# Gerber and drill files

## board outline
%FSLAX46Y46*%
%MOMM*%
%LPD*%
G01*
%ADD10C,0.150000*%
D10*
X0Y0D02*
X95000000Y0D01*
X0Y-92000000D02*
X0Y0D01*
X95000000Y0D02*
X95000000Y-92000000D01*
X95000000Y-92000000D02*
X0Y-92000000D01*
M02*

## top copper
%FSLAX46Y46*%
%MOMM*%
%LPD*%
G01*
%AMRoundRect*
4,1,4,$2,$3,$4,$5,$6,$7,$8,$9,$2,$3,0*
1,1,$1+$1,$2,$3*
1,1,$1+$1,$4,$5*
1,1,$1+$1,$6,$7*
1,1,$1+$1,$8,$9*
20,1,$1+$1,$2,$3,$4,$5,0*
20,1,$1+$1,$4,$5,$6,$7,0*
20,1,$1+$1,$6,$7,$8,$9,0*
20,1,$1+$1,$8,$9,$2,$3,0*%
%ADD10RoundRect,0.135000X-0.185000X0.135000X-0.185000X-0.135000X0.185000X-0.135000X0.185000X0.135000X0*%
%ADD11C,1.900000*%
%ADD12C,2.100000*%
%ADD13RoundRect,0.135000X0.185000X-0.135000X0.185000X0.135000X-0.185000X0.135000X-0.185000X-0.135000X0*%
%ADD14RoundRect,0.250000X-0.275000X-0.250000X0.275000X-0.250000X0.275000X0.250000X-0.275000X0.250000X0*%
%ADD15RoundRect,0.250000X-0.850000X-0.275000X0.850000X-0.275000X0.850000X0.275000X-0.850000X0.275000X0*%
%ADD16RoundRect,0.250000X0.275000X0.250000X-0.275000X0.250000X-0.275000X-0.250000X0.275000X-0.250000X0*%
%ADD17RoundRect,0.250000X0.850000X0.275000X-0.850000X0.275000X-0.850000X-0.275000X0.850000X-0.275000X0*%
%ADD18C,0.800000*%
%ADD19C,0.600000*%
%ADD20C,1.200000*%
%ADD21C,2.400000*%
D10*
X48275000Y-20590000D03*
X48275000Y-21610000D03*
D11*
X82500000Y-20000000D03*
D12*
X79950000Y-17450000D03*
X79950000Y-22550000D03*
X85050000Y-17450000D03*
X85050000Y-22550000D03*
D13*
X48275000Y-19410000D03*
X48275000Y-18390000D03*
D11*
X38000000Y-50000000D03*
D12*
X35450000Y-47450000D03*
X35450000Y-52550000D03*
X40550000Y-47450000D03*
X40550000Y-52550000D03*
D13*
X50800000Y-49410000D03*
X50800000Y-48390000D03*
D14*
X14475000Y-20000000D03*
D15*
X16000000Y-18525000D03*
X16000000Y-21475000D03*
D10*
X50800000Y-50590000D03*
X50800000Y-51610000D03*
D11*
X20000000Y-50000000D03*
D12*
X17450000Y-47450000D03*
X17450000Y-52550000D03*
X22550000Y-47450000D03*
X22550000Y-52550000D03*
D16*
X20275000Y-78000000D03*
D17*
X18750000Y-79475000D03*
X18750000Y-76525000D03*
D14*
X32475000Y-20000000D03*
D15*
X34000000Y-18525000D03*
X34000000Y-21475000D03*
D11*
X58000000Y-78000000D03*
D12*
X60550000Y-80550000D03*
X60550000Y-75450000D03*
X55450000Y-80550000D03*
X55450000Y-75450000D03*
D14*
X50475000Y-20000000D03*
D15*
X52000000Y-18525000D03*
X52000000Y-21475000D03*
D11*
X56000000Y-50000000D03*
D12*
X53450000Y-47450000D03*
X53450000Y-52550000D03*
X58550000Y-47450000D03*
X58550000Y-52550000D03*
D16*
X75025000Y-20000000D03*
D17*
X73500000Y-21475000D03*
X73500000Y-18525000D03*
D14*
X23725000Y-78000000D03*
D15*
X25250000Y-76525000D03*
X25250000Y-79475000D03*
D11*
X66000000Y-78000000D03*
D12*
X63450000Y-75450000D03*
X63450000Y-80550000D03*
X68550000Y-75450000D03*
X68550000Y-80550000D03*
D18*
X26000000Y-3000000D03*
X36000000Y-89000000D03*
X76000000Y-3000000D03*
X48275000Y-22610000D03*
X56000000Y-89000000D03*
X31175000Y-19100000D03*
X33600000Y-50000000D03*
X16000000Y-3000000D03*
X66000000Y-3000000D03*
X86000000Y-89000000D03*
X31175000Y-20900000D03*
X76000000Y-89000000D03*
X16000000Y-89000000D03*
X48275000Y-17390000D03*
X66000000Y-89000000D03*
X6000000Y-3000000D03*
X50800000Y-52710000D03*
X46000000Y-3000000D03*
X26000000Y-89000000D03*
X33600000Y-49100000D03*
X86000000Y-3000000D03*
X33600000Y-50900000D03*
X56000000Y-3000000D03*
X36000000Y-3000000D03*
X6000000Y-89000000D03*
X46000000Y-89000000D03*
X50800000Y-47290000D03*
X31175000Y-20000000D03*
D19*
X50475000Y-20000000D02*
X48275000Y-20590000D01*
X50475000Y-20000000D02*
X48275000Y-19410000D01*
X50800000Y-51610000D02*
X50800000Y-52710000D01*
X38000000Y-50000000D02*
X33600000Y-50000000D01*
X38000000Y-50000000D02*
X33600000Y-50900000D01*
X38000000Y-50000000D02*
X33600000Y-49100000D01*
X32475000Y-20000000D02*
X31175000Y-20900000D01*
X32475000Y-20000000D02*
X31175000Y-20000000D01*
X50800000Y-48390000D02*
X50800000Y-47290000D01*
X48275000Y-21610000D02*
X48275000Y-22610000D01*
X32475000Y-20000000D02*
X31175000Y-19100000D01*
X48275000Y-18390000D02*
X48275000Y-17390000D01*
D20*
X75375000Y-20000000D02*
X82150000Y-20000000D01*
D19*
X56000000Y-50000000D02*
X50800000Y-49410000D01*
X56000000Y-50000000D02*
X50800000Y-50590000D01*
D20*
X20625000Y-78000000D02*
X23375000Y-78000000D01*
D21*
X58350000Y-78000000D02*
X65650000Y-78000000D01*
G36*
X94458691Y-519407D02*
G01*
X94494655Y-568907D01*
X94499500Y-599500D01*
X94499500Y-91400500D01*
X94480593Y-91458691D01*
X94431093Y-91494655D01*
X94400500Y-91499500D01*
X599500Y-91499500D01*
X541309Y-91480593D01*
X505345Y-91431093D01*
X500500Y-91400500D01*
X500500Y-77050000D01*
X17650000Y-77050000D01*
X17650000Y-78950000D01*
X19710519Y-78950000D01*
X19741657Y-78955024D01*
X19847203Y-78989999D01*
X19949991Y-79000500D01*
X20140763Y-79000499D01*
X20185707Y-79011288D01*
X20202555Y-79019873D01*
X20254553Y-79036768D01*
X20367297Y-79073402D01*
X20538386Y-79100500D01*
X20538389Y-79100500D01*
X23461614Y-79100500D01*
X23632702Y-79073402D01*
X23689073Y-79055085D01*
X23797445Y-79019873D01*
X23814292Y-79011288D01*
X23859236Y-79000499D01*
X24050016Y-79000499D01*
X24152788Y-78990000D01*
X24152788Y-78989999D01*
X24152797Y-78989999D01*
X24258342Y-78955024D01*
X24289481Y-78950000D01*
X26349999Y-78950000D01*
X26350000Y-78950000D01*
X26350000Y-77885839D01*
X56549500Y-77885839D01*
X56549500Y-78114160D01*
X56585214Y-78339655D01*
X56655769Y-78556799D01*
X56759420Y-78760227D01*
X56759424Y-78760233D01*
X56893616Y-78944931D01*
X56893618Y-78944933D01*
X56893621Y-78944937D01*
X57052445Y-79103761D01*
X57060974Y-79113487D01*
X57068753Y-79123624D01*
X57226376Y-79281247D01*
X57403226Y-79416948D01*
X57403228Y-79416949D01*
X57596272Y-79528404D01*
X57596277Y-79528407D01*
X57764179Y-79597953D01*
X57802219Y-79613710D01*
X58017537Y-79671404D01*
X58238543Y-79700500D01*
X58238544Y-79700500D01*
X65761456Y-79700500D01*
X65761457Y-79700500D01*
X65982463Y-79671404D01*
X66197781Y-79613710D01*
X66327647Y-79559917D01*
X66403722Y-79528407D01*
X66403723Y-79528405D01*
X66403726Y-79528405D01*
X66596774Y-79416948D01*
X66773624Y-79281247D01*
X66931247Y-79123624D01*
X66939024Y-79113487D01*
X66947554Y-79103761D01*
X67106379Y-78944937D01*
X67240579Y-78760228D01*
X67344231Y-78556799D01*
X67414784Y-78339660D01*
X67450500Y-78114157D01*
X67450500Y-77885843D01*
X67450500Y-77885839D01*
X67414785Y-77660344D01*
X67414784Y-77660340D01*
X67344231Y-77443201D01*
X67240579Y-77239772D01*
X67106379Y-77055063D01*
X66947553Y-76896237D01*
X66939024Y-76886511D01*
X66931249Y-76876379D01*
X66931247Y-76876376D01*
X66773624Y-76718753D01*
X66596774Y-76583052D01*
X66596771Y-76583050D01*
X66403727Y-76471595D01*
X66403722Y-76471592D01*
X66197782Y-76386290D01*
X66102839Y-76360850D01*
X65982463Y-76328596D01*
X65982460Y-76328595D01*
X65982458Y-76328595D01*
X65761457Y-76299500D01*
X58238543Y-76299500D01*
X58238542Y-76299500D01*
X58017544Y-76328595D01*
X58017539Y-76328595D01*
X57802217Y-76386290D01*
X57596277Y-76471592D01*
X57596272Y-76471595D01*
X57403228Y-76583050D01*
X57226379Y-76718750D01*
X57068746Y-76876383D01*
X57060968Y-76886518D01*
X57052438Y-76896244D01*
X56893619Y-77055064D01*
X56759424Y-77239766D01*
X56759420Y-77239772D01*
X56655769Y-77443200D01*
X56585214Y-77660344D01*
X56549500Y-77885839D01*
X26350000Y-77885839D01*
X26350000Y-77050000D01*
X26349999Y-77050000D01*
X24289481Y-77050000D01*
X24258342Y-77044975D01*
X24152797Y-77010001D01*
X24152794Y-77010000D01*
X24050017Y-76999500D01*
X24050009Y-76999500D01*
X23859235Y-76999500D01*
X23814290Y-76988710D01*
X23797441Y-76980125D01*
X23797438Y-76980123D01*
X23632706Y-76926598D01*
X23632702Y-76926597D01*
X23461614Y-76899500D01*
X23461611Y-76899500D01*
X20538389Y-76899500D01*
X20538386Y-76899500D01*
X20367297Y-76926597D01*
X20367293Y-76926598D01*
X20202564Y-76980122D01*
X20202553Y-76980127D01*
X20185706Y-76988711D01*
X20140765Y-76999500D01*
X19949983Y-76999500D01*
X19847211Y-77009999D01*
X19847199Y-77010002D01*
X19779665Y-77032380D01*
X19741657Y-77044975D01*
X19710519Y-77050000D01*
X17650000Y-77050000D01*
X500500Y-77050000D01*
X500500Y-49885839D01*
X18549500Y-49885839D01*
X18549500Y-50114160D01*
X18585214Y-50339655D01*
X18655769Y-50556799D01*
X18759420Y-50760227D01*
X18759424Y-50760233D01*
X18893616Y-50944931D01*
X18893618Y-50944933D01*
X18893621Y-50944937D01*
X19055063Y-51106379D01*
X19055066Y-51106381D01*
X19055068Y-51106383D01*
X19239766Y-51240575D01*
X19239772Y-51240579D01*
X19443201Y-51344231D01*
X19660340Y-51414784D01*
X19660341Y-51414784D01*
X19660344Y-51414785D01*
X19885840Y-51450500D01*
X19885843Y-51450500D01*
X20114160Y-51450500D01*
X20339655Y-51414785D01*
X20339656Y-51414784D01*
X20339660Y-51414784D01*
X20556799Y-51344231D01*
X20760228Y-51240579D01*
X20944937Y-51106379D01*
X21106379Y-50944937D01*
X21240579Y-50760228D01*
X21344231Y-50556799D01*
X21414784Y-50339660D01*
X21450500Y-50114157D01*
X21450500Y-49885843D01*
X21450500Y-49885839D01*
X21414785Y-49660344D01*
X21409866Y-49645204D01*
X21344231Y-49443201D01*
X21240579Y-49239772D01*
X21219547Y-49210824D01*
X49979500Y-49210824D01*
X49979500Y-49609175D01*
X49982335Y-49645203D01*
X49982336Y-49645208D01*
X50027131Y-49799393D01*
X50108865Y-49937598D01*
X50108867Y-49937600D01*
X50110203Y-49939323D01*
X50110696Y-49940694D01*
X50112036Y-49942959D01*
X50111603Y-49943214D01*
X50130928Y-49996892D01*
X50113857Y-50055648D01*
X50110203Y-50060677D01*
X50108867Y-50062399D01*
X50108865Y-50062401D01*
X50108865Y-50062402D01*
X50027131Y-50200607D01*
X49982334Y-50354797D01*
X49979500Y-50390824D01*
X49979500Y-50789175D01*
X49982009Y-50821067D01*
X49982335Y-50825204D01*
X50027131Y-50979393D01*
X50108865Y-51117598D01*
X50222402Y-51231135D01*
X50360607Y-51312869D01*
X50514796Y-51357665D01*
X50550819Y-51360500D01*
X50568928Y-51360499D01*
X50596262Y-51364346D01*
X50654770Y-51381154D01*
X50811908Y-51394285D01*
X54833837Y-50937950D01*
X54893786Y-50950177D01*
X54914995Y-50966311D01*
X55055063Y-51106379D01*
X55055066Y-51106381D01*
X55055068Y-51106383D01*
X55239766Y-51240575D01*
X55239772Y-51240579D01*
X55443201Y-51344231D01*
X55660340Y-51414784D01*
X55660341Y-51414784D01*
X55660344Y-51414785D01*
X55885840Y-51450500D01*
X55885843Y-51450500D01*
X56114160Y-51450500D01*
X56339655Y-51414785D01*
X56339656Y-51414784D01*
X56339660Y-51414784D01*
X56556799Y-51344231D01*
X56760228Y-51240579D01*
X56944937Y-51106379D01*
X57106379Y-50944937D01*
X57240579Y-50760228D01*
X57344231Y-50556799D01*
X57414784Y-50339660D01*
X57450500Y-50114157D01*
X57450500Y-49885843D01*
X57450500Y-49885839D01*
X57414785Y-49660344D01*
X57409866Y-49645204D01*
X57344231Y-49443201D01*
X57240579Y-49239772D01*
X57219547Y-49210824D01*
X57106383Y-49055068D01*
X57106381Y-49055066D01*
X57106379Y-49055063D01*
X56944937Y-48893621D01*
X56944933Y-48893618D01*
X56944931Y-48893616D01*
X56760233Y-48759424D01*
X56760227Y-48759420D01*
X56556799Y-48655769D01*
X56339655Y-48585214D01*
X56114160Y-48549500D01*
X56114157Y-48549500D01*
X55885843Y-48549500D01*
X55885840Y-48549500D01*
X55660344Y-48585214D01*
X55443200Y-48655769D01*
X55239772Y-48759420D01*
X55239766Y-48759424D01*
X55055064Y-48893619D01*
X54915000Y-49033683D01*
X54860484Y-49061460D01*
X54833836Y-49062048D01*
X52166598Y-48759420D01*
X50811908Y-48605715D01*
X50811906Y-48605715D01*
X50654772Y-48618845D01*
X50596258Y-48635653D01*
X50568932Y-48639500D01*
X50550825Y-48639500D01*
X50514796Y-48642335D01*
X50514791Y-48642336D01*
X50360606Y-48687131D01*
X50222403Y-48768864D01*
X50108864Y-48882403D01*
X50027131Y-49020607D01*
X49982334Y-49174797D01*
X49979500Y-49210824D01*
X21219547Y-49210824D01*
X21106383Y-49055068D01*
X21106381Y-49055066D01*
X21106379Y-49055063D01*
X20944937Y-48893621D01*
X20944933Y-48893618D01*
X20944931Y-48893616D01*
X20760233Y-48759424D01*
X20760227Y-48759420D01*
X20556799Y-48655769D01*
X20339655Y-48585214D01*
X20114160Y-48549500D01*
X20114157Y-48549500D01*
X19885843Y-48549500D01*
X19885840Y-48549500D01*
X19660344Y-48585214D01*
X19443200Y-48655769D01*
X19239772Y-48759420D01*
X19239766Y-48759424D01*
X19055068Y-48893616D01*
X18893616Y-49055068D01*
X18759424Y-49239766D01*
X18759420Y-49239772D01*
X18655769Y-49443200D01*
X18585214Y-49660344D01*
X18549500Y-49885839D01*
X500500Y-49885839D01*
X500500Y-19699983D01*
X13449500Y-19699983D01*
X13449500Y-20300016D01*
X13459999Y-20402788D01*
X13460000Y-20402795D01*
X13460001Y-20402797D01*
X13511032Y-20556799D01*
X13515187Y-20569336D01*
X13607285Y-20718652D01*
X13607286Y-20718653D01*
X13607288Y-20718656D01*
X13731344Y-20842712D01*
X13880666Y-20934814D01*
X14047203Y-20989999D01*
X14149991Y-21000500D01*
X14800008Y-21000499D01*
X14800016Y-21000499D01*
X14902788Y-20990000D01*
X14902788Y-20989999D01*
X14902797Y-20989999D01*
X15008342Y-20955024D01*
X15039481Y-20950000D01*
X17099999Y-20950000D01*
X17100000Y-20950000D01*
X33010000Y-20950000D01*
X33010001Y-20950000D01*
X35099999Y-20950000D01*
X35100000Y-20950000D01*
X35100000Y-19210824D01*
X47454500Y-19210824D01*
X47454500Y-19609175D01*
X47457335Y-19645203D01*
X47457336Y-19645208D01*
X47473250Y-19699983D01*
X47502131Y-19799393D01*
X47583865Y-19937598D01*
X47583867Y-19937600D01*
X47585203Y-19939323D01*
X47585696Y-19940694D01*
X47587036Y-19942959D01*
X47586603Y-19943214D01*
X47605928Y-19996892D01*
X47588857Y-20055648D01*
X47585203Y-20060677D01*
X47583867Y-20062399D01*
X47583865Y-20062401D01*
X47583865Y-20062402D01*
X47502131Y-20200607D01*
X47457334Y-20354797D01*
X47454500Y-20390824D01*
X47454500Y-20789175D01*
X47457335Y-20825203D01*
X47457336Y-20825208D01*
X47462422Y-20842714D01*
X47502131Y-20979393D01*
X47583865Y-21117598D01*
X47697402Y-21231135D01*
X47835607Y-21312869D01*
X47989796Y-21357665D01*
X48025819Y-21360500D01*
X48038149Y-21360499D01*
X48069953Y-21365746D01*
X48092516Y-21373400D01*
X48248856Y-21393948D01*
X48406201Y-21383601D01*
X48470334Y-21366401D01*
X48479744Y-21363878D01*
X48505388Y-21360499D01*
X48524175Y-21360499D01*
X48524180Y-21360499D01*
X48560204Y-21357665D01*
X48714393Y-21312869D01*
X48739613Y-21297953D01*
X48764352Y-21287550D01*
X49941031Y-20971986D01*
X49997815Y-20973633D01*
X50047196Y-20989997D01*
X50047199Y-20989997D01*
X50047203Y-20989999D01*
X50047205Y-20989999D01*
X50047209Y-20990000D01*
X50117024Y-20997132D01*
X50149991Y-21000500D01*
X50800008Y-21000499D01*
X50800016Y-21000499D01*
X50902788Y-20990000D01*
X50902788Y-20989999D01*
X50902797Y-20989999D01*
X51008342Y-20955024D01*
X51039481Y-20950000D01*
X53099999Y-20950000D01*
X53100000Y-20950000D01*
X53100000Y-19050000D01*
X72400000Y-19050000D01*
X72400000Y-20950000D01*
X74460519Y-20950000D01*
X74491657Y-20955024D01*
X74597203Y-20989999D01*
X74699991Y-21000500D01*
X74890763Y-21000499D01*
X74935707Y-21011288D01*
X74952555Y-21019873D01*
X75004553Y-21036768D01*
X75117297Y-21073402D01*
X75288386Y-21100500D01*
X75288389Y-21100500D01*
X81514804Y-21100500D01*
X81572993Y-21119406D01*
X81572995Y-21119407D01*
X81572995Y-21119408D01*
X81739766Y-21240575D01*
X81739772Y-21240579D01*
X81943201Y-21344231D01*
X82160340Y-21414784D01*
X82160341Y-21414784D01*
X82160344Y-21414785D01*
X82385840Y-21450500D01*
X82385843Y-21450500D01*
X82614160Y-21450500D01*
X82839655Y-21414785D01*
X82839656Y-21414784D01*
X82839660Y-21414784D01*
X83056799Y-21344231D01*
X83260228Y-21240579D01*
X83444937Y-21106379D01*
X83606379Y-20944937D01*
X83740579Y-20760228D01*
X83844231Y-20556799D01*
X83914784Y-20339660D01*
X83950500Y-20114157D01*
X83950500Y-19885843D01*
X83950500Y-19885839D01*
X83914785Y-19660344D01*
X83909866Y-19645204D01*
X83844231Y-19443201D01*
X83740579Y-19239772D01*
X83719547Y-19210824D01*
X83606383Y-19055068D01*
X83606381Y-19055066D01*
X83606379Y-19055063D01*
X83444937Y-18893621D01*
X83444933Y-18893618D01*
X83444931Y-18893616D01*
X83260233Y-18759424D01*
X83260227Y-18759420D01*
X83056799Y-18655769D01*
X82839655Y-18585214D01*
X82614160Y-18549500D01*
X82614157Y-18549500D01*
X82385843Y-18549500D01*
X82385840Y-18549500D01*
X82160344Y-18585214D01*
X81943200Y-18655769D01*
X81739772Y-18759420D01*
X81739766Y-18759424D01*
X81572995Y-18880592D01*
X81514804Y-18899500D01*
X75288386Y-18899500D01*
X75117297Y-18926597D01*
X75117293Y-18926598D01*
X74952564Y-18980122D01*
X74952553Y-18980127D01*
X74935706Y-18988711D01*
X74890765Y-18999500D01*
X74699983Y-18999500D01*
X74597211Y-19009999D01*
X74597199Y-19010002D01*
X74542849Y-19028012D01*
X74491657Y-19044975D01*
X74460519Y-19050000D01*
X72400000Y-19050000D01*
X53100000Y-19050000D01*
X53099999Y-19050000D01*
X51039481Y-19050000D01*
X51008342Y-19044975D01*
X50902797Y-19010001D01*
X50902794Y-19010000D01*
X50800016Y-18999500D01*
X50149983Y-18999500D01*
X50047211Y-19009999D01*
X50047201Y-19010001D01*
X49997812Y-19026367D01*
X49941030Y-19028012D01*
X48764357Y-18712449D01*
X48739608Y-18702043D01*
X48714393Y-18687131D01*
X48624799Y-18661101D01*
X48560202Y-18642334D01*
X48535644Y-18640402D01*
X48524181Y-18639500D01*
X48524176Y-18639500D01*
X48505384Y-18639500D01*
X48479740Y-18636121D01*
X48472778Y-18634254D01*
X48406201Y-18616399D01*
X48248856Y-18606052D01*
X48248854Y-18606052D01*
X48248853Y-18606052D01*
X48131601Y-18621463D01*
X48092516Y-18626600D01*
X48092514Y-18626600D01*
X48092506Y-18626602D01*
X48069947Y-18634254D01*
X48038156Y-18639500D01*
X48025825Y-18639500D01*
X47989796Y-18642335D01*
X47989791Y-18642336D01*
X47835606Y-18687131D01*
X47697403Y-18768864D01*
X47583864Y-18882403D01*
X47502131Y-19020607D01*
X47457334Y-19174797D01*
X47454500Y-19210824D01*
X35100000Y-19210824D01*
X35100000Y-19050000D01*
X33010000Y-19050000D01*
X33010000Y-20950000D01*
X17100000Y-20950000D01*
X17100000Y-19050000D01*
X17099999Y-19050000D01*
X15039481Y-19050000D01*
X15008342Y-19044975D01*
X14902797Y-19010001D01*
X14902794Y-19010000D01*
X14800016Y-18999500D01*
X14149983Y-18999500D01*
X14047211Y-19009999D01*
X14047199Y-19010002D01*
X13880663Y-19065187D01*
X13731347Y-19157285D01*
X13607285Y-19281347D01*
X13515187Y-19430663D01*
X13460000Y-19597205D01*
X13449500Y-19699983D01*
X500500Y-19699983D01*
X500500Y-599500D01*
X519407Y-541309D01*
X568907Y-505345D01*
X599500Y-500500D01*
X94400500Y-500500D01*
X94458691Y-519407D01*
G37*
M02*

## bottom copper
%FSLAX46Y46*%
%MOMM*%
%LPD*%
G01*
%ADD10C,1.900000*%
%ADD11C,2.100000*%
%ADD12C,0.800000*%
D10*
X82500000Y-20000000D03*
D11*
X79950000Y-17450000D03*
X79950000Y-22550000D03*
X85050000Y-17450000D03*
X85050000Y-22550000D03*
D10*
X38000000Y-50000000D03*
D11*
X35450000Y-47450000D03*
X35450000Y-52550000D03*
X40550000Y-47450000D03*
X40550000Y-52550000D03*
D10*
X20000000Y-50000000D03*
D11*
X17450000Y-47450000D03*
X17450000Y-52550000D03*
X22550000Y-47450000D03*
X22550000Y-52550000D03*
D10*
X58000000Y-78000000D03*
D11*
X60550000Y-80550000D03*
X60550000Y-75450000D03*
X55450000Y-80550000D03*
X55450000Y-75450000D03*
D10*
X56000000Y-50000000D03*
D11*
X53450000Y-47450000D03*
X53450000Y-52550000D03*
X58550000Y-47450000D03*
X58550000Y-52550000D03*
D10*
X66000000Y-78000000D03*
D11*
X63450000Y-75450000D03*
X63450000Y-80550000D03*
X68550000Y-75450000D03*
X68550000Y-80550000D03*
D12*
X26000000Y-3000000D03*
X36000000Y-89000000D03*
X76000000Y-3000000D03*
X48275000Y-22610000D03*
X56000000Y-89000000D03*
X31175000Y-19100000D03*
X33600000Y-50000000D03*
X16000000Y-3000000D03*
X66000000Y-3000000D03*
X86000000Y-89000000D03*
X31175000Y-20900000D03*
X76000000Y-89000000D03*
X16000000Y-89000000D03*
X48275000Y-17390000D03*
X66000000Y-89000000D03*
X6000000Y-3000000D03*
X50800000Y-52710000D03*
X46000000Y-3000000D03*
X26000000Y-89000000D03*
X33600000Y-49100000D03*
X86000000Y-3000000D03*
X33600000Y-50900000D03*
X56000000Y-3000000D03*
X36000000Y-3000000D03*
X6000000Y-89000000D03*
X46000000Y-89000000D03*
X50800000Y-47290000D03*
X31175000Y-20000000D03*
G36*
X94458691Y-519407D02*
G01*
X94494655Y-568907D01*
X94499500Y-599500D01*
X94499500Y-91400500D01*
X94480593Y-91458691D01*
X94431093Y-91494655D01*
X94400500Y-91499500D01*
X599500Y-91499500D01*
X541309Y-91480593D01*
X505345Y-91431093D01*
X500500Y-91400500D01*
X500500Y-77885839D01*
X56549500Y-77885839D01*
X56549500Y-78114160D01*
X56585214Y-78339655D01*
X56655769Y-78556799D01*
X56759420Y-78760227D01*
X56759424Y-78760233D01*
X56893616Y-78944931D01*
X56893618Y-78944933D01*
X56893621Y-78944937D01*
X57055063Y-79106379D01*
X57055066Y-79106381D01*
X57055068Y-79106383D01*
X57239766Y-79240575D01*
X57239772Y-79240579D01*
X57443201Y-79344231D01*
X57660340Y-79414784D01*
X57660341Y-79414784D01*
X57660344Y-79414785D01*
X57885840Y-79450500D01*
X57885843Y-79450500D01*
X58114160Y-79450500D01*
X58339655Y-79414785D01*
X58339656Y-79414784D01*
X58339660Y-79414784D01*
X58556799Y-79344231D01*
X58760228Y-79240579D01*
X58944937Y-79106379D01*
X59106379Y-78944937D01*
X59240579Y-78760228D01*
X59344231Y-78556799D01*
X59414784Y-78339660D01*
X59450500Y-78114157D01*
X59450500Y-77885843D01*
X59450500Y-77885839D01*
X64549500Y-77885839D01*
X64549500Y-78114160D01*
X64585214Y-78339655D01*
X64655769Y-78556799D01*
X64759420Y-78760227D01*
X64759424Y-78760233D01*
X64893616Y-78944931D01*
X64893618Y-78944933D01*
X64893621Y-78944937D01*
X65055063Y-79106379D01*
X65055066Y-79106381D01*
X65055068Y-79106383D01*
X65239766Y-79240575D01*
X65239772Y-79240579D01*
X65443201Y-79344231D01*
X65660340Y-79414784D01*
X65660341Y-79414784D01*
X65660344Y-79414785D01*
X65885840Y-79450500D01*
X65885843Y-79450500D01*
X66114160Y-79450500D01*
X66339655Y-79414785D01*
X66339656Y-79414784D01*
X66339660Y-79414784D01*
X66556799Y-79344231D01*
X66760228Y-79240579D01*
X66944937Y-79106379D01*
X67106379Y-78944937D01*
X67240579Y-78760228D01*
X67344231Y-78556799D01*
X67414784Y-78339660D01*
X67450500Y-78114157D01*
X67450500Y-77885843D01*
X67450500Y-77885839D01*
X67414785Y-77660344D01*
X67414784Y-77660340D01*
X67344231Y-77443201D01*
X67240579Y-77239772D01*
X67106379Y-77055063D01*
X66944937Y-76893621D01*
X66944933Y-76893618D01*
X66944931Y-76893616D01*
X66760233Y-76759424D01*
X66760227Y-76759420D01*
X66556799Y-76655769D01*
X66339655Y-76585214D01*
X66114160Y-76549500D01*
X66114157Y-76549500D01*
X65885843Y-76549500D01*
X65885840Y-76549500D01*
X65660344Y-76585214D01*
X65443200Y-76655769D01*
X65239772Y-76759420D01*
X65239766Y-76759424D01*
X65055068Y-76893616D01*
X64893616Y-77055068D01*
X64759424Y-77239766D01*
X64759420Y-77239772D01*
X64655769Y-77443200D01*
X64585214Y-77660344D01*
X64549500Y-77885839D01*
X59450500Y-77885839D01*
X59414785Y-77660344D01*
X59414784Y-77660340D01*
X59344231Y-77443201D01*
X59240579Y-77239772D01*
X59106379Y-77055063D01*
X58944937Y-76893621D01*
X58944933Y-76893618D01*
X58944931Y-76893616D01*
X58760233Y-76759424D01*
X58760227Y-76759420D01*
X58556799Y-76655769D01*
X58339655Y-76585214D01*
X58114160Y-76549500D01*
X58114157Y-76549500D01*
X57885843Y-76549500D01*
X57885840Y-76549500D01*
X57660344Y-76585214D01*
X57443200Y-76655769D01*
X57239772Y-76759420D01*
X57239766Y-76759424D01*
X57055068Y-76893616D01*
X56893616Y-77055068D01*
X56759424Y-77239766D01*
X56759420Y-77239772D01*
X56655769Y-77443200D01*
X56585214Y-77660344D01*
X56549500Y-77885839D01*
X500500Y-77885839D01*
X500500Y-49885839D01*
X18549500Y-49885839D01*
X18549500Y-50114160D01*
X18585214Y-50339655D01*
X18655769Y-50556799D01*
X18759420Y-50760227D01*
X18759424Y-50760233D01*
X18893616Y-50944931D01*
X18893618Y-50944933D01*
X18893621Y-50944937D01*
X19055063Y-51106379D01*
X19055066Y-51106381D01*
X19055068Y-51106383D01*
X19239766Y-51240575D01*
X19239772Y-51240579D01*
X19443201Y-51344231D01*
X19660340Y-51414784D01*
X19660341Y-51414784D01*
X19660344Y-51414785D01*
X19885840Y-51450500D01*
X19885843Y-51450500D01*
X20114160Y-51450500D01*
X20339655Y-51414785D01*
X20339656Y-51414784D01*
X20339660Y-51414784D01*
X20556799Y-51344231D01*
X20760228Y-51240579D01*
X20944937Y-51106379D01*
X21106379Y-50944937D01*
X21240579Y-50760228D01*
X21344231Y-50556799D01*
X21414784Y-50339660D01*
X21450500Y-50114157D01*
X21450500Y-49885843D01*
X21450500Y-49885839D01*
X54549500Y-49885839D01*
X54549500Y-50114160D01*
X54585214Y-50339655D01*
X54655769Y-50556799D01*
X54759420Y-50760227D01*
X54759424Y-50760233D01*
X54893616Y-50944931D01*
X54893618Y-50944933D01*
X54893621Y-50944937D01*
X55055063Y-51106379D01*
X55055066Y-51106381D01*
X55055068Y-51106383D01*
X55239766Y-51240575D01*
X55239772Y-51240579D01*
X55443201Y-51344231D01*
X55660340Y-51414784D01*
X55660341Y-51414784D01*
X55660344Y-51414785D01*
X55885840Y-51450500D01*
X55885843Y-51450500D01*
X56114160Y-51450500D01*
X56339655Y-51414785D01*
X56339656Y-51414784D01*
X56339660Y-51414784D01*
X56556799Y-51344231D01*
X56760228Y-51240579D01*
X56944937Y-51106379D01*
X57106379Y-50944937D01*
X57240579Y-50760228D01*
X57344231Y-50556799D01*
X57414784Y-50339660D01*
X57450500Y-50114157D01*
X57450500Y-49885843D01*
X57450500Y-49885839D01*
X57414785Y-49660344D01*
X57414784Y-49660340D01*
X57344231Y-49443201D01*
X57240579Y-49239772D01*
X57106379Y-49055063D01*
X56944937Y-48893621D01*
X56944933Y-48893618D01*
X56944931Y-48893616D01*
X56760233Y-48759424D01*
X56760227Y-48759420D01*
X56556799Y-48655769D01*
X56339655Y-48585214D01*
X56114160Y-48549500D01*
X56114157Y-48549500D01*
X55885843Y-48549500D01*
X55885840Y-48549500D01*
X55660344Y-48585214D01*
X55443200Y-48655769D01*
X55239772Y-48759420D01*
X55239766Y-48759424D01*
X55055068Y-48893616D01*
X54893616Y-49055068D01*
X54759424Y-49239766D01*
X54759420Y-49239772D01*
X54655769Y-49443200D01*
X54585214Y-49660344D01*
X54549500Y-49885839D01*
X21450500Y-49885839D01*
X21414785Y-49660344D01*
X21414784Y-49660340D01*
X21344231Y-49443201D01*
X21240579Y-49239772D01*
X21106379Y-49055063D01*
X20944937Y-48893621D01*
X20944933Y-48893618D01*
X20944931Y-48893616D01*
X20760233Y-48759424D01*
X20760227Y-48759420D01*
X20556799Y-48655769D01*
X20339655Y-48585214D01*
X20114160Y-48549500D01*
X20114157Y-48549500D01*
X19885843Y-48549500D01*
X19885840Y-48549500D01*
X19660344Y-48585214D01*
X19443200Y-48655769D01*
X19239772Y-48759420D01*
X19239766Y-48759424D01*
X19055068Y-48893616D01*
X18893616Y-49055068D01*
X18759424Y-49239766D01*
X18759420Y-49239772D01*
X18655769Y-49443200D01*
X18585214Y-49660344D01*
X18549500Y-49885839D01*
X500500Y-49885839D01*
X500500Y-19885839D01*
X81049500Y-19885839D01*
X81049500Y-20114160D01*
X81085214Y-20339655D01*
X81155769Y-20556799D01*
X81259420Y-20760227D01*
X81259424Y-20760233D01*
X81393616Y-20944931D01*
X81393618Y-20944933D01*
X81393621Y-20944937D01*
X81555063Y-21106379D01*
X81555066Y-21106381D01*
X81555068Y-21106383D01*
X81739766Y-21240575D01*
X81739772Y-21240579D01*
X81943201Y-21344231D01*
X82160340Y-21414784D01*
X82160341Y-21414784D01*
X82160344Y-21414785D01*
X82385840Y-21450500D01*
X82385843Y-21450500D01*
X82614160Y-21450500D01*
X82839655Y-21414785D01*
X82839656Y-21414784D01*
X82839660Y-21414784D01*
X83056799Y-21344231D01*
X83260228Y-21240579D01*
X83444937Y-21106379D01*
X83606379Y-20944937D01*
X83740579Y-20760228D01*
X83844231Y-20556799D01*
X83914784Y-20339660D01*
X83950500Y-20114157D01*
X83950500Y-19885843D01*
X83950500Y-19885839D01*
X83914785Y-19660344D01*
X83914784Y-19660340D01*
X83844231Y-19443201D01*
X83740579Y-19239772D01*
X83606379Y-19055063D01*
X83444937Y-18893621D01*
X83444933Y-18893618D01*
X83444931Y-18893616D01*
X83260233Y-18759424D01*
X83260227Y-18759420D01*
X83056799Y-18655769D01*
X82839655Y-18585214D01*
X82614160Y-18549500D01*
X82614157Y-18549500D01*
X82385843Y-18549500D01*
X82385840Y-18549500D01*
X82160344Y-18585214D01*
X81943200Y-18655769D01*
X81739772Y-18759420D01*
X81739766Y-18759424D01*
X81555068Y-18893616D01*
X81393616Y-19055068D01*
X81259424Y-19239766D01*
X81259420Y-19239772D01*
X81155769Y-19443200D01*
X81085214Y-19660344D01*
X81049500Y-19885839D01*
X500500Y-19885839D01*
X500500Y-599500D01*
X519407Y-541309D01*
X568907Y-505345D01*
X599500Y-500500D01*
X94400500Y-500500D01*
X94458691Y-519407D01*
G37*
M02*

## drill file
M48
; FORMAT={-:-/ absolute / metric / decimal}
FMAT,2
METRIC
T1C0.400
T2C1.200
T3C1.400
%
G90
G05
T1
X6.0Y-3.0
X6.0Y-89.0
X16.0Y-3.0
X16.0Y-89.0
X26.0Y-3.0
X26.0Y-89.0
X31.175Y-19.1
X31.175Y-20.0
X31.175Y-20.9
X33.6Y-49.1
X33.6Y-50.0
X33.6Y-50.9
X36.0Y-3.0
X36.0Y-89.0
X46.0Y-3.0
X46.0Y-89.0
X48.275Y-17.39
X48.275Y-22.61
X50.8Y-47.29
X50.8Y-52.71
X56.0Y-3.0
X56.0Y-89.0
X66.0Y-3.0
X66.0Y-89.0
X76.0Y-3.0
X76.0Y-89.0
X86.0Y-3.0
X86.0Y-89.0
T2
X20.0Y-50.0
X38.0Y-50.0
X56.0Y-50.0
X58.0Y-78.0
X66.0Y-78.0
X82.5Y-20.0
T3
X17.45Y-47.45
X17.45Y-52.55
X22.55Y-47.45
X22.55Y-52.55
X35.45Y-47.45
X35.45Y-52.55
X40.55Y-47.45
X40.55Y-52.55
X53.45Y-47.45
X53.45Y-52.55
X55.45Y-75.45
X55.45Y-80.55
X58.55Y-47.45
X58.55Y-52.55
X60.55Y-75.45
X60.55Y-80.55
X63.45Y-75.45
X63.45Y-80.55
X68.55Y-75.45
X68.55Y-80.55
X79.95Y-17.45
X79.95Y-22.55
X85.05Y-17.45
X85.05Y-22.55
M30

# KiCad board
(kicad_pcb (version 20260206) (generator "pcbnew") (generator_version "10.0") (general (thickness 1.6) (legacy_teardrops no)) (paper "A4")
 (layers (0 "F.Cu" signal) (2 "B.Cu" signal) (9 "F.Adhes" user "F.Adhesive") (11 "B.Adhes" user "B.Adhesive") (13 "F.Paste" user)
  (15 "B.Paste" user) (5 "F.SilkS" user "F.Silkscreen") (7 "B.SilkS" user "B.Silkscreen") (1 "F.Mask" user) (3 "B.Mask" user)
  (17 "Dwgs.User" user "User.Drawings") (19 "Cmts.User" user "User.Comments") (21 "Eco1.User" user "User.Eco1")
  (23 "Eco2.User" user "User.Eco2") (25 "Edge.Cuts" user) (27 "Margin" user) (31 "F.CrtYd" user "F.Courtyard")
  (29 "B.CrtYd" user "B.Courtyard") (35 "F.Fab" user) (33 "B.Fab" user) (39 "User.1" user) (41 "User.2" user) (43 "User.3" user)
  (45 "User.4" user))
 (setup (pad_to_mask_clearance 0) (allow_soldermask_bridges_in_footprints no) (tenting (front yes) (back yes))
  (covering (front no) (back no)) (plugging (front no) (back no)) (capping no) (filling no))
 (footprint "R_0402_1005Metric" (layer "F.Cu") (at 48.275 21.1 -90)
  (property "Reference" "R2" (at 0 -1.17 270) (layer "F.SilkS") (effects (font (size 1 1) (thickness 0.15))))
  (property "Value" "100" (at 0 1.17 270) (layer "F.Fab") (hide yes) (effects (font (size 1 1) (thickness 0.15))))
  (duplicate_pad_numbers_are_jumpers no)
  (pad "1" smd roundrect (at -0.51 0 270) (size 0.54 0.64) (layers "F.Cu" "F.Mask" "F.Paste") (roundrect_rratio 0.25) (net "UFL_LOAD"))
  (pad "2" smd roundrect (at 0.51 0 270) (size 0.54 0.64) (layers "F.Cu" "F.Mask" "F.Paste") (roundrect_rratio 0.25) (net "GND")))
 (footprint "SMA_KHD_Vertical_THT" (layer "F.Cu") (at 82.5 20)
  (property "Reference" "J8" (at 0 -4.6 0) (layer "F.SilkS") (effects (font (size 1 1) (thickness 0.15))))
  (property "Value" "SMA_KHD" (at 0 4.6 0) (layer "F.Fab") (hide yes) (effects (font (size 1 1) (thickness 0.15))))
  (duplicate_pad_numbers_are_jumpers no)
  (pad "1" thru_hole circle (at 0 0) (size 1.9 1.9) (drill 1.2) (layers "*.Cu" "*.Mask") (remove_unused_layers no) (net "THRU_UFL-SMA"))
  (pad "2" thru_hole circle (at -2.55 -2.55) (size 2.1 2.1) (drill 1.4) (layers "*.Cu" "*.Mask") (remove_unused_layers no) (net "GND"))
  (pad "2" thru_hole circle (at -2.55 2.55) (size 2.1 2.1) (drill 1.4) (layers "*.Cu" "*.Mask") (remove_unused_layers no) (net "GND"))
  (pad "2" thru_hole circle (at 2.55 -2.55) (size 2.1 2.1) (drill 1.4) (layers "*.Cu" "*.Mask") (remove_unused_layers no) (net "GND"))
  (pad "2" thru_hole circle (at 2.55 2.55) (size 2.1 2.1) (drill 1.4) (layers "*.Cu" "*.Mask") (remove_unused_layers no) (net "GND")))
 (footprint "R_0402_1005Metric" (layer "F.Cu") (at 48.275 18.9 90)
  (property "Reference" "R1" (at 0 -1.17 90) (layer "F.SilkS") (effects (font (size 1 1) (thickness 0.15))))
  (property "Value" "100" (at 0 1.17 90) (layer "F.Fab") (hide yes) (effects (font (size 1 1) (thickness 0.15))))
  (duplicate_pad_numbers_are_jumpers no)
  (pad "1" smd roundrect (at -0.51 0 90) (size 0.54 0.64) (layers "F.Cu" "F.Mask" "F.Paste") (roundrect_rratio 0.25) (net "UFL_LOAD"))
  (pad "2" smd roundrect (at 0.51 0 90) (size 0.54 0.64) (layers "F.Cu" "F.Mask" "F.Paste") (roundrect_rratio 0.25) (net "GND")))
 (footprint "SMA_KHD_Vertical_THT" (layer "F.Cu") (at 38 50)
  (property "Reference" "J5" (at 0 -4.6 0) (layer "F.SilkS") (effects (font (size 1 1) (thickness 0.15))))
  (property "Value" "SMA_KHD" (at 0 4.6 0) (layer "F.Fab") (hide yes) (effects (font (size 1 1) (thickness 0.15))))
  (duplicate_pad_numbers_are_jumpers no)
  (pad "1" thru_hole circle (at 0 0) (size 1.9 1.9) (drill 1.2) (layers "*.Cu" "*.Mask") (remove_unused_layers no) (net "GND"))
  (pad "2" thru_hole circle (at -2.55 -2.55) (size 2.1 2.1) (drill 1.4) (layers "*.Cu" "*.Mask") (remove_unused_layers no) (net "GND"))
  (pad "2" thru_hole circle (at -2.55 2.55) (size 2.1 2.1) (drill 1.4) (layers "*.Cu" "*.Mask") (remove_unused_layers no) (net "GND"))
  (pad "2" thru_hole circle (at 2.55 -2.55) (size 2.1 2.1) (drill 1.4) (layers "*.Cu" "*.Mask") (remove_unused_layers no) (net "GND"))
  (pad "2" thru_hole circle (at 2.55 2.55) (size 2.1 2.1) (drill 1.4) (layers "*.Cu" "*.Mask") (remove_unused_layers no) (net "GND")))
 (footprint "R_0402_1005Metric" (layer "F.Cu") (at 50.8 48.9 90)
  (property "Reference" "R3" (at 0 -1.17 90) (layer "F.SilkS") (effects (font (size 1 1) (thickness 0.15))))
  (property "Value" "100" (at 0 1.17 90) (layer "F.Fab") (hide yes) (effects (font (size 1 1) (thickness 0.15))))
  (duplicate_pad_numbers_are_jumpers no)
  (pad "1" smd roundrect (at -0.51 0 90) (size 0.54 0.64) (layers "F.Cu" "F.Mask" "F.Paste") (roundrect_rratio 0.25) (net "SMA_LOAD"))
  (pad "2" smd roundrect (at 0.51 0 90) (size 0.54 0.64) (layers "F.Cu" "F.Mask" "F.Paste") (roundrect_rratio 0.25) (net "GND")))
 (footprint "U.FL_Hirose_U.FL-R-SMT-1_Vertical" (layer "F.Cu") (at 16 20)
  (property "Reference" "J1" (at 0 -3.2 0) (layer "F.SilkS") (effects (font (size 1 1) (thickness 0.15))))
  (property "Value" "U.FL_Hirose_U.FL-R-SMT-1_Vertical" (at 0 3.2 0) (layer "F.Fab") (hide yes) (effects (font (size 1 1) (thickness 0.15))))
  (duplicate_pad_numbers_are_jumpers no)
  (pad "1" smd roundrect (at -1.525 0) (size 1.05 1) (layers "F.Cu" "F.Mask" "F.Paste") (roundrect_rratio 0.25) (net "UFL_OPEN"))
  (pad "2" smd roundrect (at 0 -1.475) (size 2.2 1.05) (layers "F.Cu" "F.Mask" "F.Paste") (roundrect_rratio 0.2380952381) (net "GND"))
  (pad "2" smd roundrect (at 0 1.475) (size 2.2 1.05) (layers "F.Cu" "F.Mask" "F.Paste") (roundrect_rratio 0.2380952381) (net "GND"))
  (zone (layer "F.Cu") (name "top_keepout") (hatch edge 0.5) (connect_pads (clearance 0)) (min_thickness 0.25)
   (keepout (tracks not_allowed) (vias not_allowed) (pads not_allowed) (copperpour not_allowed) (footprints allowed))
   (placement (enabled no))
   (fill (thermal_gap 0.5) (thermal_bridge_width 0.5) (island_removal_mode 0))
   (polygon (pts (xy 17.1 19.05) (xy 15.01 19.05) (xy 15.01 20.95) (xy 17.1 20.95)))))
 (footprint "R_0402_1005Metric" (layer "F.Cu") (at 50.8 51.1 -90)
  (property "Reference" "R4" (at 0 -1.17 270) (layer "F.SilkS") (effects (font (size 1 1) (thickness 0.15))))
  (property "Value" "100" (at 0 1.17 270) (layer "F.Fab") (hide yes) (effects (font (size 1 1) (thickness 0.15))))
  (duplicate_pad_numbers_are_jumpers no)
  (pad "1" smd roundrect (at -0.51 0 270) (size 0.54 0.64) (layers "F.Cu" "F.Mask" "F.Paste") (roundrect_rratio 0.25) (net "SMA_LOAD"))
  (pad "2" smd roundrect (at 0.51 0 270) (size 0.54 0.64) (layers "F.Cu" "F.Mask" "F.Paste") (roundrect_rratio 0.25) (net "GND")))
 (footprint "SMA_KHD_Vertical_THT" (layer "F.Cu") (at 20 50)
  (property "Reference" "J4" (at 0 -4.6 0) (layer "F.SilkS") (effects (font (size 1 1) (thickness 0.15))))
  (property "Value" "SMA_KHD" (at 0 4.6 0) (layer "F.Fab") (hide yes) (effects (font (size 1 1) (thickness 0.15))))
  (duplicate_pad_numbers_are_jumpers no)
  (pad "1" thru_hole circle (at 0 0) (size 1.9 1.9) (drill 1.2) (layers "*.Cu" "*.Mask") (remove_unused_layers no) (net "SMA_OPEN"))
  (pad "2" thru_hole circle (at -2.55 -2.55) (size 2.1 2.1) (drill 1.4) (layers "*.Cu" "*.Mask") (remove_unused_layers no) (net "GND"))
  (pad "2" thru_hole circle (at -2.55 2.55) (size 2.1 2.1) (drill 1.4) (layers "*.Cu" "*.Mask") (remove_unused_layers no) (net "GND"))
  (pad "2" thru_hole circle (at 2.55 -2.55) (size 2.1 2.1) (drill 1.4) (layers "*.Cu" "*.Mask") (remove_unused_layers no) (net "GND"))
  (pad "2" thru_hole circle (at 2.55 2.55) (size 2.1 2.1) (drill 1.4) (layers "*.Cu" "*.Mask") (remove_unused_layers no) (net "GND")))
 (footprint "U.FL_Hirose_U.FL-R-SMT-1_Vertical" (layer "F.Cu") (at 18.75 78 180)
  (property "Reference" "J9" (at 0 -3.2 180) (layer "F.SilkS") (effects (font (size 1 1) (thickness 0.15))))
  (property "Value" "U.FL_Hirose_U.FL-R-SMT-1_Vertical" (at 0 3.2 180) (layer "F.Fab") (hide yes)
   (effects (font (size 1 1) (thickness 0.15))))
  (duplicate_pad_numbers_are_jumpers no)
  (pad "1" smd roundrect (at -1.525 0 180) (size 1.05 1) (layers "F.Cu" "F.Mask" "F.Paste") (roundrect_rratio 0.25) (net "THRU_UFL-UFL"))
  (pad "2" smd roundrect (at 0 -1.475 180) (size 2.2 1.05) (layers "F.Cu" "F.Mask" "F.Paste") (roundrect_rratio 0.2380952381) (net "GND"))
  (pad "2" smd roundrect (at 0 1.475 180) (size 2.2 1.05) (layers "F.Cu" "F.Mask" "F.Paste") (roundrect_rratio 0.2380952381) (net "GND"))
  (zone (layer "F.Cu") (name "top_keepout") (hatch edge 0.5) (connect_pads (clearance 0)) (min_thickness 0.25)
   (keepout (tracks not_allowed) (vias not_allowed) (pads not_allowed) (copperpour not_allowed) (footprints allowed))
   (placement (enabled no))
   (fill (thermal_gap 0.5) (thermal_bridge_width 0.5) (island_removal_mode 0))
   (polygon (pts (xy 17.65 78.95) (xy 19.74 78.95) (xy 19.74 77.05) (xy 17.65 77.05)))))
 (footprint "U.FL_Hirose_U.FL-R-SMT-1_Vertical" (layer "F.Cu") (at 34 20)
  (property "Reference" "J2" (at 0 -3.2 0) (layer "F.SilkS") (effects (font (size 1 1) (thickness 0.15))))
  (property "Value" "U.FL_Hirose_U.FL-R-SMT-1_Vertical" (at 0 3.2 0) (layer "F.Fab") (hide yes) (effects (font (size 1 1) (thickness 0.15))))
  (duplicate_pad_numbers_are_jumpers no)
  (pad "1" smd roundrect (at -1.525 0) (size 1.05 1) (layers "F.Cu" "F.Mask" "F.Paste") (roundrect_rratio 0.25) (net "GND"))
  (pad "2" smd roundrect (at 0 -1.475) (size 2.2 1.05) (layers "F.Cu" "F.Mask" "F.Paste") (roundrect_rratio 0.2380952381) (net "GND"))
  (pad "2" smd roundrect (at 0 1.475) (size 2.2 1.05) (layers "F.Cu" "F.Mask" "F.Paste") (roundrect_rratio 0.2380952381) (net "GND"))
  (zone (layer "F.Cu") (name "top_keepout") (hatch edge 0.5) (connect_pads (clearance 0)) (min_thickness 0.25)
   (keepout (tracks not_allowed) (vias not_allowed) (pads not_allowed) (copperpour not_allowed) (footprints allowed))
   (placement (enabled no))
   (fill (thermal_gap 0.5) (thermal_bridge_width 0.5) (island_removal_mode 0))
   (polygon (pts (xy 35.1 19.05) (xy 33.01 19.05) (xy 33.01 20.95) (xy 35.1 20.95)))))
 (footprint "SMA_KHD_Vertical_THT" (layer "F.Cu") (at 58 78 180)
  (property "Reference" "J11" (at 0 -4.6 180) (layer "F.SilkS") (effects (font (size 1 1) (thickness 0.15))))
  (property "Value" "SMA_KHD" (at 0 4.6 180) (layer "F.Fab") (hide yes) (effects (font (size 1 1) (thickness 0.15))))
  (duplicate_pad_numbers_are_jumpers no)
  (pad "1" thru_hole circle (at 0 0 180) (size 1.9 1.9) (drill 1.2) (layers "*.Cu" "*.Mask") (remove_unused_layers no) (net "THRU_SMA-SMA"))
  (pad "2" thru_hole circle (at -2.55 -2.55 180) (size 2.1 2.1) (drill 1.4) (layers "*.Cu" "*.Mask") (remove_unused_layers no) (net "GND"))
  (pad "2" thru_hole circle (at -2.55 2.55 180) (size 2.1 2.1) (drill 1.4) (layers "*.Cu" "*.Mask") (remove_unused_layers no) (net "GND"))
  (pad "2" thru_hole circle (at 2.55 -2.55 180) (size 2.1 2.1) (drill 1.4) (layers "*.Cu" "*.Mask") (remove_unused_layers no) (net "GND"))
  (pad "2" thru_hole circle (at 2.55 2.55 180) (size 2.1 2.1) (drill 1.4) (layers "*.Cu" "*.Mask") (remove_unused_layers no) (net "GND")))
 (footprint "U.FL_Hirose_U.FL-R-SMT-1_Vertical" (layer "F.Cu") (at 52 20)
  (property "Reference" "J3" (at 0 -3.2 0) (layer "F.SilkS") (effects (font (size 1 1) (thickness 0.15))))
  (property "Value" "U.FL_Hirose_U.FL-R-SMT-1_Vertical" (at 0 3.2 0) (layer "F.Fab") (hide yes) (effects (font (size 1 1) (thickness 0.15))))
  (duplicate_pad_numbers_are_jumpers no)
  (pad "1" smd roundrect (at -1.525 0) (size 1.05 1) (layers "F.Cu" "F.Mask" "F.Paste") (roundrect_rratio 0.25) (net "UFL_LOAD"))
  (pad "2" smd roundrect (at 0 -1.475) (size 2.2 1.05) (layers "F.Cu" "F.Mask" "F.Paste") (roundrect_rratio 0.2380952381) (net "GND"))
  (pad "2" smd roundrect (at 0 1.475) (size 2.2 1.05) (layers "F.Cu" "F.Mask" "F.Paste") (roundrect_rratio 0.2380952381) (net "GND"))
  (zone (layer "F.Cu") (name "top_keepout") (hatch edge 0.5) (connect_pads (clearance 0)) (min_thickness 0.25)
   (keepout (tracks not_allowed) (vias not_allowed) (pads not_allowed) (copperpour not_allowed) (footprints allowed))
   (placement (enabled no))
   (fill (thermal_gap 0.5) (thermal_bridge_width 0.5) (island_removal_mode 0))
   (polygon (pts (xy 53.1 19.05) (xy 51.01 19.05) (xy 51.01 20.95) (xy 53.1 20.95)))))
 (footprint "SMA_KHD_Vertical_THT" (layer "F.Cu") (at 56 50)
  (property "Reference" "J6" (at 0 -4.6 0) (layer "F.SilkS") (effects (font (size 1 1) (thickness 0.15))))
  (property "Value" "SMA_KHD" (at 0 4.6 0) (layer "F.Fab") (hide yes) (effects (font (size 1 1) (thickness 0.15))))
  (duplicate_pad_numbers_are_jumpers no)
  (pad "1" thru_hole circle (at 0 0) (size 1.9 1.9) (drill 1.2) (layers "*.Cu" "*.Mask") (remove_unused_layers no) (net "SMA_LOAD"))
  (pad "2" thru_hole circle (at -2.55 -2.55) (size 2.1 2.1) (drill 1.4) (layers "*.Cu" "*.Mask") (remove_unused_layers no) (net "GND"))
  (pad "2" thru_hole circle (at -2.55 2.55) (size 2.1 2.1) (drill 1.4) (layers "*.Cu" "*.Mask") (remove_unused_layers no) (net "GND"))
  (pad "2" thru_hole circle (at 2.55 -2.55) (size 2.1 2.1) (drill 1.4) (layers "*.Cu" "*.Mask") (remove_unused_layers no) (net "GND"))
  (pad "2" thru_hole circle (at 2.55 2.55) (size 2.1 2.1) (drill 1.4) (layers "*.Cu" "*.Mask") (remove_unused_layers no) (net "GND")))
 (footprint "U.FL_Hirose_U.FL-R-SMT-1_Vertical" (layer "F.Cu") (at 73.5 20 180)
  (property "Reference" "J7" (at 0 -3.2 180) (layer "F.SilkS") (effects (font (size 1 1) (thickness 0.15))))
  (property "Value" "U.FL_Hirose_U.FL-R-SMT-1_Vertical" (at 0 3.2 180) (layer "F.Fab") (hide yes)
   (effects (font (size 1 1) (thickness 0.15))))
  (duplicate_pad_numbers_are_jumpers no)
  (pad "1" smd roundrect (at -1.525 0 180) (size 1.05 1) (layers "F.Cu" "F.Mask" "F.Paste") (roundrect_rratio 0.25) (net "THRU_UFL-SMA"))
  (pad "2" smd roundrect (at 0 -1.475 180) (size 2.2 1.05) (layers "F.Cu" "F.Mask" "F.Paste") (roundrect_rratio 0.2380952381) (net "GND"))
  (pad "2" smd roundrect (at 0 1.475 180) (size 2.2 1.05) (layers "F.Cu" "F.Mask" "F.Paste") (roundrect_rratio 0.2380952381) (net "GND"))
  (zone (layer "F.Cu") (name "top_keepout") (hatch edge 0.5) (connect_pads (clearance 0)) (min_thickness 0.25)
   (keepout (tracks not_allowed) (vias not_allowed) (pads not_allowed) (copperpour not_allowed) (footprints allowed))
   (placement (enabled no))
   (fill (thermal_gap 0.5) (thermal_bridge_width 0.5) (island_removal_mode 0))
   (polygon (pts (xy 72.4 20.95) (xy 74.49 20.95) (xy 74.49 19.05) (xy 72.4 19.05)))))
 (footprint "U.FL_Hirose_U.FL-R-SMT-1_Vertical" (layer "F.Cu") (at 25.25 78)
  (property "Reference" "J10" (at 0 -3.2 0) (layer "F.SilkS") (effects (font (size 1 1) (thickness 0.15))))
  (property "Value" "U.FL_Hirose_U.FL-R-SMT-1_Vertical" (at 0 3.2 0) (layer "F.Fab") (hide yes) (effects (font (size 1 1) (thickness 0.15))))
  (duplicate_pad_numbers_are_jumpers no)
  (pad "1" smd roundrect (at -1.525 0) (size 1.05 1) (layers "F.Cu" "F.Mask" "F.Paste") (roundrect_rratio 0.25) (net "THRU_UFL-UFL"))
  (pad "2" smd roundrect (at 0 -1.475) (size 2.2 1.05) (layers "F.Cu" "F.Mask" "F.Paste") (roundrect_rratio 0.2380952381) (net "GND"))
  (pad "2" smd roundrect (at 0 1.475) (size 2.2 1.05) (layers "F.Cu" "F.Mask" "F.Paste") (roundrect_rratio 0.2380952381) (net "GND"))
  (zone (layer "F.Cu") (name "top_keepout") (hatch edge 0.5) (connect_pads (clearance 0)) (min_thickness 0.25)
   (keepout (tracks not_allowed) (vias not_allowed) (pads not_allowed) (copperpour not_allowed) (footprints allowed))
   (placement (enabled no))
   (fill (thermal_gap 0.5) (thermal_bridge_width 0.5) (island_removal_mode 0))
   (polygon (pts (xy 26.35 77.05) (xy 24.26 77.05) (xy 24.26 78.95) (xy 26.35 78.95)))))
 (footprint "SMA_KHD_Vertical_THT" (layer "F.Cu") (at 66 78)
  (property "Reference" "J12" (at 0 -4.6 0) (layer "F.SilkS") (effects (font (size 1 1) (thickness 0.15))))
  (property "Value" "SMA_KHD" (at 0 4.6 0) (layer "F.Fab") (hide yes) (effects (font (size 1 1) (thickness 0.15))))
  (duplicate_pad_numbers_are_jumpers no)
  (pad "1" thru_hole circle (at 0 0) (size 1.9 1.9) (drill 1.2) (layers "*.Cu" "*.Mask") (remove_unused_layers no) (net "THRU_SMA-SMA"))
  (pad "2" thru_hole circle (at -2.55 -2.55) (size 2.1 2.1) (drill 1.4) (layers "*.Cu" "*.Mask") (remove_unused_layers no) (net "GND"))
  (pad "2" thru_hole circle (at -2.55 2.55) (size 2.1 2.1) (drill 1.4) (layers "*.Cu" "*.Mask") (remove_unused_layers no) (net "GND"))
  (pad "2" thru_hole circle (at 2.55 -2.55) (size 2.1 2.1) (drill 1.4) (layers "*.Cu" "*.Mask") (remove_unused_layers no) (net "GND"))
  (pad "2" thru_hole circle (at 2.55 2.55) (size 2.1 2.1) (drill 1.4) (layers "*.Cu" "*.Mask") (remove_unused_layers no) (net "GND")))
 (gr_line (start 0 0) (end 95 0) (stroke (width 0.15) (type default)) (layer "Edge.Cuts"))
 (gr_line (start 0 92) (end 0 0) (stroke (width 0.15) (type default)) (layer "Edge.Cuts"))
 (gr_line (start 95 0) (end 95 92) (stroke (width 0.15) (type default)) (layer "Edge.Cuts"))
 (gr_line (start 95 92) (end 0 92) (stroke (width 0.15) (type default)) (layer "Edge.Cuts"))
 (segment (start 50.475 20) (end 48.275 20.59) (width 0.6) (layer "F.Cu") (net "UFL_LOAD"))
 (segment (start 50.475 20) (end 48.275 19.41) (width 0.6) (layer "F.Cu") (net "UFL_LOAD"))
 (segment (start 50.8 51.61) (end 50.8 52.71) (width 0.6) (layer "F.Cu") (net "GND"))
 (segment (start 38 50) (end 33.6 50) (width 0.6) (layer "F.Cu") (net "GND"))
 (segment (start 38 50) (end 33.6 50.9) (width 0.6) (layer "F.Cu") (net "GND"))
 (segment (start 38 50) (end 33.6 49.1) (width 0.6) (layer "F.Cu") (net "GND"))
 (segment (start 32.475 20) (end 31.175 20.9) (width 0.6) (layer "F.Cu") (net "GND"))
 (segment (start 32.475 20) (end 31.175 20) (width 0.6) (layer "F.Cu") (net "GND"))
 (segment (start 50.8 48.39) (end 50.8 47.29) (width 0.6) (layer "F.Cu") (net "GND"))
 (segment (start 48.275 21.61) (end 48.275 22.61) (width 0.6) (layer "F.Cu") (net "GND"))
 (segment (start 32.475 20) (end 31.175 19.1) (width 0.6) (layer "F.Cu") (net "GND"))
 (segment (start 48.275 18.39) (end 48.275 17.39) (width 0.6) (layer "F.Cu") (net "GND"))
 (via (at 26 3) (size 0.8) (drill 0.4) (layers "F.Cu" "B.Cu") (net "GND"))
 (via (at 36 89) (size 0.8) (drill 0.4) (layers "F.Cu" "B.Cu") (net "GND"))
 (via (at 76 3) (size 0.8) (drill 0.4) (layers "F.Cu" "B.Cu") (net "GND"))
 (via (at 48.275 22.61) (size 0.8) (drill 0.4) (layers "F.Cu" "B.Cu") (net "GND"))
 (via (at 56 89) (size 0.8) (drill 0.4) (layers "F.Cu" "B.Cu") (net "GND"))
 (via (at 31.175 19.1) (size 0.8) (drill 0.4) (layers "F.Cu" "B.Cu") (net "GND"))
 (via (at 33.6 50) (size 0.8) (drill 0.4) (layers "F.Cu" "B.Cu") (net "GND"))
 (via (at 16 3) (size 0.8) (drill 0.4) (layers "F.Cu" "B.Cu") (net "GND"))
 (via (at 66 3) (size 0.8) (drill 0.4) (layers "F.Cu" "B.Cu") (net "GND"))
 (via (at 86 89) (size 0.8) (drill 0.4) (layers "F.Cu" "B.Cu") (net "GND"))
 (via (at 31.175 20.9) (size 0.8) (drill 0.4) (layers "F.Cu" "B.Cu") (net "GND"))
 (via (at 76 89) (size 0.8) (drill 0.4) (layers "F.Cu" "B.Cu") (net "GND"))
 (via (at 16 89) (size 0.8) (drill 0.4) (layers "F.Cu" "B.Cu") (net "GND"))
 (via (at 48.275 17.39) (size 0.8) (drill 0.4) (layers "F.Cu" "B.Cu") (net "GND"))
 (via (at 66 89) (size 0.8) (drill 0.4) (layers "F.Cu" "B.Cu") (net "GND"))
 (via (at 6 3) (size 0.8) (drill 0.4) (layers "F.Cu" "B.Cu") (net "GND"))
 (via (at 50.8 52.71) (size 0.8) (drill 0.4) (layers "F.Cu" "B.Cu") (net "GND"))
 (via (at 46 3) (size 0.8) (drill 0.4) (layers "F.Cu" "B.Cu") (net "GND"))
 (via (at 26 89) (size 0.8) (drill 0.4) (layers "F.Cu" "B.Cu") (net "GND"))
 (via (at 33.6 49.1) (size 0.8) (drill 0.4) (layers "F.Cu" "B.Cu") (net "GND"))
 (via (at 86 3) (size 0.8) (drill 0.4) (layers "F.Cu" "B.Cu") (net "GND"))
 (via (at 33.6 50.9) (size 0.8) (drill 0.4) (layers "F.Cu" "B.Cu") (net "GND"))
 (via (at 56 3) (size 0.8) (drill 0.4) (layers "F.Cu" "B.Cu") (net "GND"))
 (via (at 36 3) (size 0.8) (drill 0.4) (layers "F.Cu" "B.Cu") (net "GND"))
 (via (at 6 89) (size 0.8) (drill 0.4) (layers "F.Cu" "B.Cu") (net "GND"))
 (via (at 46 89) (size 0.8) (drill 0.4) (layers "F.Cu" "B.Cu") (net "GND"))
 (via (at 50.8 47.29) (size 0.8) (drill 0.4) (layers "F.Cu" "B.Cu") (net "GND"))
 (via (at 31.175 20) (size 0.8) (drill 0.4) (layers "F.Cu" "B.Cu") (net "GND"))
 (segment (start 75.375 20) (end 82.15 20) (width 1.2) (layer "F.Cu") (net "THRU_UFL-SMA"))
 (segment (start 56 50) (end 50.8 49.41) (width 0.6) (layer "F.Cu") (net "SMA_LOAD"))
 (segment (start 56 50) (end 50.8 50.59) (width 0.6) (layer "F.Cu") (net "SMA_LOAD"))
 (segment (start 20.625 78) (end 23.375 78) (width 1.2) (layer "F.Cu") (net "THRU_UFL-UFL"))
 (segment (start 58.35 78) (end 65.65 78) (width 2.4) (layer "F.Cu") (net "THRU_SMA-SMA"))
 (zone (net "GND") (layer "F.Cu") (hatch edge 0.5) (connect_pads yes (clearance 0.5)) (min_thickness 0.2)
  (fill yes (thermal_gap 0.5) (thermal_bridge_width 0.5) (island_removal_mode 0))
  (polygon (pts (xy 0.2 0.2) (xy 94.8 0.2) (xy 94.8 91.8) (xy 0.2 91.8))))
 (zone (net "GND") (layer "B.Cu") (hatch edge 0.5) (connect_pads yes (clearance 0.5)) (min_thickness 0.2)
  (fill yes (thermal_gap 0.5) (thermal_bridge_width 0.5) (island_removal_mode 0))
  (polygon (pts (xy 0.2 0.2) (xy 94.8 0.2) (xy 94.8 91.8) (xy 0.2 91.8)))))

